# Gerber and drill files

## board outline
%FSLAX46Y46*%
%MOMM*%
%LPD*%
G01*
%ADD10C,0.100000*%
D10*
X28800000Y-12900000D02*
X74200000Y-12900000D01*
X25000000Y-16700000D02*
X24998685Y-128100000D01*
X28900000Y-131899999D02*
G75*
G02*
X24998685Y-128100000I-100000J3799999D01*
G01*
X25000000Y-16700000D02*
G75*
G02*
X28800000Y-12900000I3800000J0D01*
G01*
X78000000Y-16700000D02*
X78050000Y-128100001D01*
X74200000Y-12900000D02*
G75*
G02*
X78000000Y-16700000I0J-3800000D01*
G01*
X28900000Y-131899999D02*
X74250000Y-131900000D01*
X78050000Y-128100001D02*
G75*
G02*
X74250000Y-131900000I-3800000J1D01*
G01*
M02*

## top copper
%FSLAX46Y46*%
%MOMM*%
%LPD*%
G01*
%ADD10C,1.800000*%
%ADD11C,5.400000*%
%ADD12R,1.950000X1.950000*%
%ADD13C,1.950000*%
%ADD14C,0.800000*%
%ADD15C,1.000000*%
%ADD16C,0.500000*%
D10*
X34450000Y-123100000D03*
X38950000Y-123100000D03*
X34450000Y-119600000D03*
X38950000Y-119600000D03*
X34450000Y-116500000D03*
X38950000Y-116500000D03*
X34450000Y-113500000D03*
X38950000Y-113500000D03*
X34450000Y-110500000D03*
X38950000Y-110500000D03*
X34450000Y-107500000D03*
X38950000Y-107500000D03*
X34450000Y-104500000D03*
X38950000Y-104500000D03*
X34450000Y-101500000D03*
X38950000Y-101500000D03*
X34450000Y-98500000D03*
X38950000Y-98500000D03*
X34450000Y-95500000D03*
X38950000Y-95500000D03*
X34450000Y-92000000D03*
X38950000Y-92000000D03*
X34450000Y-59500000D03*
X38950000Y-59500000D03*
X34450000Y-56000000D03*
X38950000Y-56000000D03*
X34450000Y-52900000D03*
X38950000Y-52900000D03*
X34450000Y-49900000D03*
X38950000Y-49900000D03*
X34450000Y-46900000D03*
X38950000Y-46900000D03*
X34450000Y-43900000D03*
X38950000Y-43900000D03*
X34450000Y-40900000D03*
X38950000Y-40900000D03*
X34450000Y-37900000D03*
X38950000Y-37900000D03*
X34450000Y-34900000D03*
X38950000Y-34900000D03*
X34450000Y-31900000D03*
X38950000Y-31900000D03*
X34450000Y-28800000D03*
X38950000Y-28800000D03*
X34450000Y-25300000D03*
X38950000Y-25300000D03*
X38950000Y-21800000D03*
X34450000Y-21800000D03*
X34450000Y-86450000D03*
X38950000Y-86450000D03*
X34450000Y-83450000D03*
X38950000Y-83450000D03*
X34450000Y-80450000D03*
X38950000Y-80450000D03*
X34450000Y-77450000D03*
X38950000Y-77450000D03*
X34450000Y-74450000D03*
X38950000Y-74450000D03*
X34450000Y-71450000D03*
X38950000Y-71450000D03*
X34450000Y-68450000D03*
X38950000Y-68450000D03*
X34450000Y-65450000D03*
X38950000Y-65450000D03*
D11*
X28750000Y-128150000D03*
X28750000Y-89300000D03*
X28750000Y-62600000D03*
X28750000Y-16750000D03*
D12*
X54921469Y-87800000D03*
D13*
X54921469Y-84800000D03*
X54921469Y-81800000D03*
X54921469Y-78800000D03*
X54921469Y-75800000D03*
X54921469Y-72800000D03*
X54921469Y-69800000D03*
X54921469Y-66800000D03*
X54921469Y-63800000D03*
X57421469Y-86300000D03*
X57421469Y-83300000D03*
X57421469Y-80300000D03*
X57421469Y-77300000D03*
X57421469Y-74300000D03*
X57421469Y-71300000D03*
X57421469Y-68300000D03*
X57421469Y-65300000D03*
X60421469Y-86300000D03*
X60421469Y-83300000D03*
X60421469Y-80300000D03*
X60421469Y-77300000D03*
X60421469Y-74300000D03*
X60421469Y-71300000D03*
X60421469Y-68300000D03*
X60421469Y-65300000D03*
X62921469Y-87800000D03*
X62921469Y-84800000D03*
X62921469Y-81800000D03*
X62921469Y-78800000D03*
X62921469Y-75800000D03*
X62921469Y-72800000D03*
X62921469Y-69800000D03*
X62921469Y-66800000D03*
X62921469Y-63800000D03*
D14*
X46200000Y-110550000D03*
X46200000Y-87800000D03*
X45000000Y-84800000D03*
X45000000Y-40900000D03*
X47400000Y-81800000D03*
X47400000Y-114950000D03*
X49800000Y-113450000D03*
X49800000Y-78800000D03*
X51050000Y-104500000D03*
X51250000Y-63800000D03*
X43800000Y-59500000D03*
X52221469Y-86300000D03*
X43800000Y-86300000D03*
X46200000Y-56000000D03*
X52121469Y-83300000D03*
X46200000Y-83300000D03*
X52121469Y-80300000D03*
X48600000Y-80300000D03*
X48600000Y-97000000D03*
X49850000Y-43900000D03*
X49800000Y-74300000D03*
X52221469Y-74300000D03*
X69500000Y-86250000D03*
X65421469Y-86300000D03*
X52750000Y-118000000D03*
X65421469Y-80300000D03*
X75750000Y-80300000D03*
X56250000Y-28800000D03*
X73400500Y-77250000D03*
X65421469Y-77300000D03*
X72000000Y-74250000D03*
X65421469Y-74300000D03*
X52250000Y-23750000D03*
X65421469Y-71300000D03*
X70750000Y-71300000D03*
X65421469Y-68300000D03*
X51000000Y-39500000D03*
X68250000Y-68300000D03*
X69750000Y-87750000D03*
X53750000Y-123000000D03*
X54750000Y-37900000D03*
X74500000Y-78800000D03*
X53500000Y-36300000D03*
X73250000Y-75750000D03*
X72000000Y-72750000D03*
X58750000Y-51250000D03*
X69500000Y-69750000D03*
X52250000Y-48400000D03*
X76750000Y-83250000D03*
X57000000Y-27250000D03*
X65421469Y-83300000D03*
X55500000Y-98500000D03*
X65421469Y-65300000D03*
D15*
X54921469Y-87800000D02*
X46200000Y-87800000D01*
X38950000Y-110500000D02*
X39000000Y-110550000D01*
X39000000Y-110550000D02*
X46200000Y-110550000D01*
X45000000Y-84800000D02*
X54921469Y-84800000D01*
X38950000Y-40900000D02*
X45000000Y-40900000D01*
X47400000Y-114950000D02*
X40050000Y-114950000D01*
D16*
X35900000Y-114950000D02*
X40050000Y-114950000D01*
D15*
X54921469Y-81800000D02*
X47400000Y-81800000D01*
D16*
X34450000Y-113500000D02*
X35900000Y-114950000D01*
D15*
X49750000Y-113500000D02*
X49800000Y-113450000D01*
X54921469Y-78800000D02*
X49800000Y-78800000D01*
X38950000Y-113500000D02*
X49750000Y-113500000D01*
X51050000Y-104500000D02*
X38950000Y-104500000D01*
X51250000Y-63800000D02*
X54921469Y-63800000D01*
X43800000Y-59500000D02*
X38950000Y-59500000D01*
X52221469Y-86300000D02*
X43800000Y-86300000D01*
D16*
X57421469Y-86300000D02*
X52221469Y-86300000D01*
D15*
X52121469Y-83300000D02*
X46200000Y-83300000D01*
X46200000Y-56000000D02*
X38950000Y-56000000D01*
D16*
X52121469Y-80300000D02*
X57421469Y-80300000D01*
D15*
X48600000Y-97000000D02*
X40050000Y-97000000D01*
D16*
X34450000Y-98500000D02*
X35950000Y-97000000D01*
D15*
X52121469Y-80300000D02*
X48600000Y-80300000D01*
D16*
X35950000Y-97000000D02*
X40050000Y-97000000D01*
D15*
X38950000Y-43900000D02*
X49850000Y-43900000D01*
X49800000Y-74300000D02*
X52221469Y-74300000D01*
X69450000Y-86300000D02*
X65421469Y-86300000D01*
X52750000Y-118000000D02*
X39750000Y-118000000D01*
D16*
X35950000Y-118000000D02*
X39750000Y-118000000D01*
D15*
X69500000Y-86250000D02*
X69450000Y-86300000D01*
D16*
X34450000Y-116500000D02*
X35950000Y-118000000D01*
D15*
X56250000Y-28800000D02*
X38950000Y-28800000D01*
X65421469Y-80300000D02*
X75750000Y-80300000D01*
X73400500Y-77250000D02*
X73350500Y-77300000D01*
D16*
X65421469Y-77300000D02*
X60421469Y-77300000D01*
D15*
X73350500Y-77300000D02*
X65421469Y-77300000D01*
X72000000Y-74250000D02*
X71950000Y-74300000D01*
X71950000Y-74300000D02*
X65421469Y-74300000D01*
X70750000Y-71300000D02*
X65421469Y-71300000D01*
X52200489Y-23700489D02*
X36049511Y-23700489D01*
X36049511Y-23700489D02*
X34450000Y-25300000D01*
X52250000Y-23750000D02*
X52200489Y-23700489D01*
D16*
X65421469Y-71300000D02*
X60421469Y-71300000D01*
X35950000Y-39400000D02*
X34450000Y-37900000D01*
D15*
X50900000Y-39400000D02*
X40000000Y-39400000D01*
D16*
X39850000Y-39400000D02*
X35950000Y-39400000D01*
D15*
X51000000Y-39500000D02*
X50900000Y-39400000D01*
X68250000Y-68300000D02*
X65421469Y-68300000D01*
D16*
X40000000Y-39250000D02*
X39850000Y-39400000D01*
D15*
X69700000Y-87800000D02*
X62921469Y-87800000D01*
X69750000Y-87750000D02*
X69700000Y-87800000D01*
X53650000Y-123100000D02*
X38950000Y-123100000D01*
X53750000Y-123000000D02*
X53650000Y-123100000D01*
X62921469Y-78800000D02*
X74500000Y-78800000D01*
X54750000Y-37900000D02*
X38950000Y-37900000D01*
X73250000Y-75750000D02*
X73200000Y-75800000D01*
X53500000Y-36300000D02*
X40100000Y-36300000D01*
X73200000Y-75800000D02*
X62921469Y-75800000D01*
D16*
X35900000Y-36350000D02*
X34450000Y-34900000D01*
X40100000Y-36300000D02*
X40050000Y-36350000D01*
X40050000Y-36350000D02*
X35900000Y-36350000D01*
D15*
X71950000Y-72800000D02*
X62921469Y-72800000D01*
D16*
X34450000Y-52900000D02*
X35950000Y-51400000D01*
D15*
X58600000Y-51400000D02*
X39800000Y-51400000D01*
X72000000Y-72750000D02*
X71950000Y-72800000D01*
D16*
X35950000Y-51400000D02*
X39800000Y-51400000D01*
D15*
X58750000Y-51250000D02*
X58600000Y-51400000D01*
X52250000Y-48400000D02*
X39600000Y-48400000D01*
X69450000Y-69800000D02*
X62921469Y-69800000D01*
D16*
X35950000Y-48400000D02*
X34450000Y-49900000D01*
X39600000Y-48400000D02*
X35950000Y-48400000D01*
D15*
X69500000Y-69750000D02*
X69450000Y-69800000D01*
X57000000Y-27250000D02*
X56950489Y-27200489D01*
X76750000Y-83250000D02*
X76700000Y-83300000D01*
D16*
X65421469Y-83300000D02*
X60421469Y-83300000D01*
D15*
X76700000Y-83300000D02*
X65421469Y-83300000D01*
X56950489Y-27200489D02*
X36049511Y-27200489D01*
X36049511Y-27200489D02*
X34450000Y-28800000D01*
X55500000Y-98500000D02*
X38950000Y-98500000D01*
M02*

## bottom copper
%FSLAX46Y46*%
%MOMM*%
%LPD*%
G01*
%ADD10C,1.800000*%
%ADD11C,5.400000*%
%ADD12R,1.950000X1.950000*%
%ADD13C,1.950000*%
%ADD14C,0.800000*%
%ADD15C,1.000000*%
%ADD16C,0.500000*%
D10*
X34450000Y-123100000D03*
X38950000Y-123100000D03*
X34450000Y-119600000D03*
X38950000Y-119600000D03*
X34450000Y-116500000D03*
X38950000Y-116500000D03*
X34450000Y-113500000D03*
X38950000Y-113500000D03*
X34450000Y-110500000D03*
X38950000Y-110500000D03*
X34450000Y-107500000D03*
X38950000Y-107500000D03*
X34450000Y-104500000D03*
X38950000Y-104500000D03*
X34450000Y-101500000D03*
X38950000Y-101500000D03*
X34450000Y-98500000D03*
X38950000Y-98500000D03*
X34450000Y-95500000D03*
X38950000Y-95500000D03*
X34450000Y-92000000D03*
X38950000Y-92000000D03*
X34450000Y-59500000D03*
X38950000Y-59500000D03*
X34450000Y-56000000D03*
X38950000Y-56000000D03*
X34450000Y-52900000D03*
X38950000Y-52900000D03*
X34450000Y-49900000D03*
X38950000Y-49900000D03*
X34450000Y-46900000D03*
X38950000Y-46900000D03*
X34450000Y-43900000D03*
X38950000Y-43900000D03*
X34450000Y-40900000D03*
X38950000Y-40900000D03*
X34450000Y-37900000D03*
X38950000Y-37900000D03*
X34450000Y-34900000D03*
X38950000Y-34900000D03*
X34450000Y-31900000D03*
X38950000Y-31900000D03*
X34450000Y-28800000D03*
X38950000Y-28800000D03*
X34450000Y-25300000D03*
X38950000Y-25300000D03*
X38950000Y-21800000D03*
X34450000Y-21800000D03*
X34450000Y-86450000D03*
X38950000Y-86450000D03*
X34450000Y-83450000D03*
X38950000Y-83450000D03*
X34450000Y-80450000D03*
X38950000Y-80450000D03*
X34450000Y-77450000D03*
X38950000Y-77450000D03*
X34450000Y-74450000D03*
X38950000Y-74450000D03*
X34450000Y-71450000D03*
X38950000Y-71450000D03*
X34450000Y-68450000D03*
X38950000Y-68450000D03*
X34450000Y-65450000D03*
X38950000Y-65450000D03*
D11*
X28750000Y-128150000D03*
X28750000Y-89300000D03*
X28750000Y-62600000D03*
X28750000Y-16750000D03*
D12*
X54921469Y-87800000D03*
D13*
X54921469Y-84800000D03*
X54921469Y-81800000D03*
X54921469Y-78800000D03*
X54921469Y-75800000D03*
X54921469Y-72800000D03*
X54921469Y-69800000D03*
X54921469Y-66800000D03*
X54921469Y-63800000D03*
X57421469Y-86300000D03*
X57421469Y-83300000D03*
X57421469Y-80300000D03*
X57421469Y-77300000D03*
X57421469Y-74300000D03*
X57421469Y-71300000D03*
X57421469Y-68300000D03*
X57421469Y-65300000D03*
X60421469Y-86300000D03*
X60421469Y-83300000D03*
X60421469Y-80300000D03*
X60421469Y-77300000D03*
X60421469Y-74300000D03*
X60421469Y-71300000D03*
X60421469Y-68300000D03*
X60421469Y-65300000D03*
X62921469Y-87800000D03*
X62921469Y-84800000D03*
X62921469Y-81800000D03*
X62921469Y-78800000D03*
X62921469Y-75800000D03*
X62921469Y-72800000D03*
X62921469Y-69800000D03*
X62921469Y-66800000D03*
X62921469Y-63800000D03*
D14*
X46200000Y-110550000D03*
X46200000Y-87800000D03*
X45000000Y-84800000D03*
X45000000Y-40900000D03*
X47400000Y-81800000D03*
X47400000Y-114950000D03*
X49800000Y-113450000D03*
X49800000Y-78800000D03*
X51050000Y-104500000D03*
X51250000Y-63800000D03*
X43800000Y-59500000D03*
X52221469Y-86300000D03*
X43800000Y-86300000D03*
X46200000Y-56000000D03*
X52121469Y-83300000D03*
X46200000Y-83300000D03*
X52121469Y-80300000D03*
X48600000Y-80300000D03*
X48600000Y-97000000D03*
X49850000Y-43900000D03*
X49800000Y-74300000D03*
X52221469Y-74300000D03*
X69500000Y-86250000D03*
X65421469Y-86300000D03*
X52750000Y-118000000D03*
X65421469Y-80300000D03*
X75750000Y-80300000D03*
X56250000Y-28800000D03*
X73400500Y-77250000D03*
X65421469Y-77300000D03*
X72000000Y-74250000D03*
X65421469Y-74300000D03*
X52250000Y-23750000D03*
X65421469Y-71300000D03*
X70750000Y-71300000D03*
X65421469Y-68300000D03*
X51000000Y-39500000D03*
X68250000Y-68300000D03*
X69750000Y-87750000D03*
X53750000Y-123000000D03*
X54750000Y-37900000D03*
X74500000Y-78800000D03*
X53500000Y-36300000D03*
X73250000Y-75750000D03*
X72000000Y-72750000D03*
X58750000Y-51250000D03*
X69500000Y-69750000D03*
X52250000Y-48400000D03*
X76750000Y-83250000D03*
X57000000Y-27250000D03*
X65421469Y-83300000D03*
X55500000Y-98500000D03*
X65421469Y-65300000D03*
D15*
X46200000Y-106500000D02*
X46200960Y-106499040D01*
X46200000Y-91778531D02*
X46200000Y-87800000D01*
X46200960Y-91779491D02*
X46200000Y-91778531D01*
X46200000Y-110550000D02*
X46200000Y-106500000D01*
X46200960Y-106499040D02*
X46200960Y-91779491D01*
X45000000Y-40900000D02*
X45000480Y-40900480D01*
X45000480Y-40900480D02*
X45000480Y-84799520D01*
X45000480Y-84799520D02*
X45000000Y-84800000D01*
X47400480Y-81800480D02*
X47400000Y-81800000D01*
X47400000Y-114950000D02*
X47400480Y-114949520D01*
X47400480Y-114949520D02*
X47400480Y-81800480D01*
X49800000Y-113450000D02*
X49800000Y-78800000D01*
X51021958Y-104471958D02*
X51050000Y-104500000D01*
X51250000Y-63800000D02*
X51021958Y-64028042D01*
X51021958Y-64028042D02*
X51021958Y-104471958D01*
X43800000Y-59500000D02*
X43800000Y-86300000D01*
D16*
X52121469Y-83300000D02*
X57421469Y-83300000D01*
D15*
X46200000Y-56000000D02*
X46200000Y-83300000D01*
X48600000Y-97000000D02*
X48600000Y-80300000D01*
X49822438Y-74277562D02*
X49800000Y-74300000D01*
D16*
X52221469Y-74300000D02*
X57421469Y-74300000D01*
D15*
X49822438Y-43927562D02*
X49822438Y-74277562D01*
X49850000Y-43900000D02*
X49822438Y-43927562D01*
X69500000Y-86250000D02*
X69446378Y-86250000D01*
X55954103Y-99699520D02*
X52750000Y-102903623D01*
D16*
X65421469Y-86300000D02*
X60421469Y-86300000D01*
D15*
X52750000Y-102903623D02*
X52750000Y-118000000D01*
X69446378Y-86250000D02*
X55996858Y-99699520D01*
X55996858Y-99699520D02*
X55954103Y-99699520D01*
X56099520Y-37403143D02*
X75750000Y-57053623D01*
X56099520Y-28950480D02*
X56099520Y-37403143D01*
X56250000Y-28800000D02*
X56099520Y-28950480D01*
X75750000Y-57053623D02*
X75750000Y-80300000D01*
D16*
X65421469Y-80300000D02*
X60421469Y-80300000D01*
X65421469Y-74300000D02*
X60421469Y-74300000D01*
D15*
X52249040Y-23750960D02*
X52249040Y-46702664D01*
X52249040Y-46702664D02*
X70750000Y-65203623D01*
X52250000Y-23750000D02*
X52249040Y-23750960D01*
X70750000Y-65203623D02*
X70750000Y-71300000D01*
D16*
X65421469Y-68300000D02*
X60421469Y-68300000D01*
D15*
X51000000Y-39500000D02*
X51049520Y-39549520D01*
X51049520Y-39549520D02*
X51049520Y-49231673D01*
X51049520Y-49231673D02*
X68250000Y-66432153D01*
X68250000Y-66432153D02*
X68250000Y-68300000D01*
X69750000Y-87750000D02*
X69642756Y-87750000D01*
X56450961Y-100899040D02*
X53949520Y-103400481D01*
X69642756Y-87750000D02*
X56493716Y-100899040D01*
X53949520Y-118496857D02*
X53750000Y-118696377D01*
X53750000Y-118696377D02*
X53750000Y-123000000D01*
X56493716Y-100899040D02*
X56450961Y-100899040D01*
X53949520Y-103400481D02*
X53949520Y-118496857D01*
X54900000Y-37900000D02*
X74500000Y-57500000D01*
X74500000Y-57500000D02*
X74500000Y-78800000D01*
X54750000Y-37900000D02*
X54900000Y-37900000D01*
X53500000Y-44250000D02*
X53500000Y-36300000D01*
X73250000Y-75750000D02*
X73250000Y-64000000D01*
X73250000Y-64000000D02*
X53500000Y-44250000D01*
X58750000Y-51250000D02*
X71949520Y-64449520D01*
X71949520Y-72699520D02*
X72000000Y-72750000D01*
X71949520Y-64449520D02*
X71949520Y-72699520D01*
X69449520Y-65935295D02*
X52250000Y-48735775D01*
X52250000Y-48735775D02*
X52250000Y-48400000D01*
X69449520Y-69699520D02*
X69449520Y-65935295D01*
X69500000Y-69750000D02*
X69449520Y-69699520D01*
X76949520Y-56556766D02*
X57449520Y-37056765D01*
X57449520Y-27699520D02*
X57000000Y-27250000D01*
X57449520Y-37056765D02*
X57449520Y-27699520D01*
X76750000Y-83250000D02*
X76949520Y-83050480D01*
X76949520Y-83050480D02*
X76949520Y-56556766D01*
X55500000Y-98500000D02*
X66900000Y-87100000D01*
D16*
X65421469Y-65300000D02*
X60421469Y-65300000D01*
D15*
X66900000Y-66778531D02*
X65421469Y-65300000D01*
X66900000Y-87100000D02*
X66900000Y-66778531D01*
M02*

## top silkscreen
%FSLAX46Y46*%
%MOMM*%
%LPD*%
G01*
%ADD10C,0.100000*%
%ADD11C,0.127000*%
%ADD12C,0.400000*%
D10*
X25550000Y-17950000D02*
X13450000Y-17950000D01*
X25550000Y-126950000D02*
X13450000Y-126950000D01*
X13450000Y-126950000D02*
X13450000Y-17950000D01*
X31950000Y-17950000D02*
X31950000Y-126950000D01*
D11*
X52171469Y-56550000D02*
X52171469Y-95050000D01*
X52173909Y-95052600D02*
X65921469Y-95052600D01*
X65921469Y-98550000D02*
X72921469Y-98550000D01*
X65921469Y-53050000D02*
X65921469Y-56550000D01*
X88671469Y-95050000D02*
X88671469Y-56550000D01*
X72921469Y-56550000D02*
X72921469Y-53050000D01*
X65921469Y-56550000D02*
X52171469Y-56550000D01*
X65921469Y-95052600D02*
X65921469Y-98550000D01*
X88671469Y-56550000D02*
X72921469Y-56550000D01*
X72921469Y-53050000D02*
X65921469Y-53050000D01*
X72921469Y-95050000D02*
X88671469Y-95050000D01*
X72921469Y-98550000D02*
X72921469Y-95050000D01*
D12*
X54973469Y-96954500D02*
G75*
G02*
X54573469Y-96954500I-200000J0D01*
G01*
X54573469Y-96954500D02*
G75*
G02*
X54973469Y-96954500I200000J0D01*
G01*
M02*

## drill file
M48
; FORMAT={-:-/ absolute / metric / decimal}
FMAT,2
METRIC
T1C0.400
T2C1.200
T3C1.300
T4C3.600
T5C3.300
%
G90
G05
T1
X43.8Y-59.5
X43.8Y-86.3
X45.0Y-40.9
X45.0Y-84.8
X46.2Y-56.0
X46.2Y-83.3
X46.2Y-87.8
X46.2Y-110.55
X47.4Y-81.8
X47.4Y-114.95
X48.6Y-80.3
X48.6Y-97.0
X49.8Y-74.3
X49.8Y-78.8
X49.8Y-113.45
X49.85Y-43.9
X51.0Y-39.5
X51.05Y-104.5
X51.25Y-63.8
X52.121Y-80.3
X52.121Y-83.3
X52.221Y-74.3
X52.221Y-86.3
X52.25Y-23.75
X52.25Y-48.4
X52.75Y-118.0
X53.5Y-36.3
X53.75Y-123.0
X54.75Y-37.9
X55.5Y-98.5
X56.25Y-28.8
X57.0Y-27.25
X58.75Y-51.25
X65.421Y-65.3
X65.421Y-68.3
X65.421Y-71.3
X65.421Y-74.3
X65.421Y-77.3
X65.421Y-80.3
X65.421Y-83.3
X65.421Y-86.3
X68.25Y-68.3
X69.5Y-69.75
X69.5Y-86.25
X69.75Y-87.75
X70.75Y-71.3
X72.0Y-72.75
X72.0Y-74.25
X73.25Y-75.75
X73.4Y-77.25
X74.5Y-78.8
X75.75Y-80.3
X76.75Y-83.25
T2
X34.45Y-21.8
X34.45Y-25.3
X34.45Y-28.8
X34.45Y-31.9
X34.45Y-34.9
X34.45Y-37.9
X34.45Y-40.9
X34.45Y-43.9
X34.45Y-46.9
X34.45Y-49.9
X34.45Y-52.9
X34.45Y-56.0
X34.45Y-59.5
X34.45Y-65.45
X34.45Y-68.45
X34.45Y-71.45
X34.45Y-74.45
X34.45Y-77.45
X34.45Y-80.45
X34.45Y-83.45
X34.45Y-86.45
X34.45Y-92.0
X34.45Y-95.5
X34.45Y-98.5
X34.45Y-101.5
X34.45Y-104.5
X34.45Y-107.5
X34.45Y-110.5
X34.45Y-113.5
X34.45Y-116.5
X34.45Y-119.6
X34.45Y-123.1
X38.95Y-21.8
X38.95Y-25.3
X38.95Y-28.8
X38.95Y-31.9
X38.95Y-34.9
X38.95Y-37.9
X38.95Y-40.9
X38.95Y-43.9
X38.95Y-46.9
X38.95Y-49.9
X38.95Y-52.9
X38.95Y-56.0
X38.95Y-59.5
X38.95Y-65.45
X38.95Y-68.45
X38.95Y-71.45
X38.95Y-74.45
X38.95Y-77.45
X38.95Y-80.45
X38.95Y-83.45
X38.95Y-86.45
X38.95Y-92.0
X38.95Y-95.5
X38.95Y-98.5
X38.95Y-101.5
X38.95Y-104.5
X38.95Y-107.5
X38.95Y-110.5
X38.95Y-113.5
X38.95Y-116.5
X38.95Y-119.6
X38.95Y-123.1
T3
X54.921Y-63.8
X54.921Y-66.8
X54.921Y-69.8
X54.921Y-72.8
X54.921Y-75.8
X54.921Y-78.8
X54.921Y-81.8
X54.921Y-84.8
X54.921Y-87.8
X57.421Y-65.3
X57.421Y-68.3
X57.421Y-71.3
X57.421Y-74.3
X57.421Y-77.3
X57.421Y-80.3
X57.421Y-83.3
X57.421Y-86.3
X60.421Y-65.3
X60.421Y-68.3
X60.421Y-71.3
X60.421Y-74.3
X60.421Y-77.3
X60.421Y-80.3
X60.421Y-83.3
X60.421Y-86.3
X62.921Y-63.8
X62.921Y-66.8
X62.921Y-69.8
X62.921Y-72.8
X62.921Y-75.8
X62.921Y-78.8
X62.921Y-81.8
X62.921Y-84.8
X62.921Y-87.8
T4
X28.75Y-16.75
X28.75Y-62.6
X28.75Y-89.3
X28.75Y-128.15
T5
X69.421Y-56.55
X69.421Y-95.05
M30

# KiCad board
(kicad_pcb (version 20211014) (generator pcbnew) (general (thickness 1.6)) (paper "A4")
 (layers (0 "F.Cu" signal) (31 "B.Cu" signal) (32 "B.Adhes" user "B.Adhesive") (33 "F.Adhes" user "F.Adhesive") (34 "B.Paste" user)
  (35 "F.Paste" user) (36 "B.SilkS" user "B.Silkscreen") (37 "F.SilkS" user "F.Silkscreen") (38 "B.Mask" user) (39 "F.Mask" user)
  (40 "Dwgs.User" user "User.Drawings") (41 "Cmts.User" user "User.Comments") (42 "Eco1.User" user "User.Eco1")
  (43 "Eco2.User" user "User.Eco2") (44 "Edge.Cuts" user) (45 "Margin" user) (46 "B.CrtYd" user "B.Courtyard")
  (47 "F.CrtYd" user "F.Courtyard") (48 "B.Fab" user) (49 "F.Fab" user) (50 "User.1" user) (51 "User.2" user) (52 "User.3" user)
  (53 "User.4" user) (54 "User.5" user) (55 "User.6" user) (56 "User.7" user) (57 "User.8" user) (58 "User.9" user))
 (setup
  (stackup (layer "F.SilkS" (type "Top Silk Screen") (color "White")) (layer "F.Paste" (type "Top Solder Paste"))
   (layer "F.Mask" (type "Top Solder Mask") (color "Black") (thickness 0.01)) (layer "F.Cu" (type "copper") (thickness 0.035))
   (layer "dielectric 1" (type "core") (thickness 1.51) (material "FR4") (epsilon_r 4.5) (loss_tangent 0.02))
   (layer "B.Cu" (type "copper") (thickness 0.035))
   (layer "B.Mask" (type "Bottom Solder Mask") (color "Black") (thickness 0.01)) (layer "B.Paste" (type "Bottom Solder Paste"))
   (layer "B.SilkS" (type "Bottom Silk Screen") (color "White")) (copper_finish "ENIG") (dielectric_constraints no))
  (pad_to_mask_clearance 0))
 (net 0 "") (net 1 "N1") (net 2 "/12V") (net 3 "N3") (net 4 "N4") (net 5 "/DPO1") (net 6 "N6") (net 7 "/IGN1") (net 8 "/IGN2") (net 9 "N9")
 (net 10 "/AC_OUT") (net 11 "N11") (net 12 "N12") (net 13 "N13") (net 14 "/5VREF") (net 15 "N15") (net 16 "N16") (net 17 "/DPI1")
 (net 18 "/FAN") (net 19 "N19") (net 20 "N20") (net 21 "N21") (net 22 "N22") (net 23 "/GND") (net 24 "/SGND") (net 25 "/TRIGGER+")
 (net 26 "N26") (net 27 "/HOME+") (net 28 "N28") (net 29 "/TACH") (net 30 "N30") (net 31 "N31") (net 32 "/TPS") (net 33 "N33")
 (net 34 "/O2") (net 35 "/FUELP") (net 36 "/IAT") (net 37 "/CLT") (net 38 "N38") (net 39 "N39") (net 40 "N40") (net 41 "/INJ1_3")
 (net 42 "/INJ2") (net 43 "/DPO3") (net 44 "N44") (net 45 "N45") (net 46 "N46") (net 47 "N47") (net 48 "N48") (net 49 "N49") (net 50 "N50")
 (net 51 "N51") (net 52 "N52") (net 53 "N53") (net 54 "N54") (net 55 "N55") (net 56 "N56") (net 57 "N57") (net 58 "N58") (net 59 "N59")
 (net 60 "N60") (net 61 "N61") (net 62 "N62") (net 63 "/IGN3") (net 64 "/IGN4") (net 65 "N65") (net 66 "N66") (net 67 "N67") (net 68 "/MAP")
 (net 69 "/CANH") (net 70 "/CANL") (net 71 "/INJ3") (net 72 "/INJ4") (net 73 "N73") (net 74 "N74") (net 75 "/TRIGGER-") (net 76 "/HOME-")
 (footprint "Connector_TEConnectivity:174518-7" (layer "F.Cu") (at 27.45 72.8 90)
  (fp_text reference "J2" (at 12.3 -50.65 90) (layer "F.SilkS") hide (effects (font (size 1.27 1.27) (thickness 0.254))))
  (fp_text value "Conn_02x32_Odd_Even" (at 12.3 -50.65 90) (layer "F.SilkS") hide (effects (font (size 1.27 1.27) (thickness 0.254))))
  (fp_line (start 54.85 -1.9) (end 54.85 -14) (layer "F.SilkS") (width 0.1))
  (fp_line (start -54.15 -1.9) (end -54.15 -14) (layer "F.SilkS") (width 0.1))
  (fp_line (start -54.15 -14) (end 54.85 -14) (layer "F.SilkS") (width 0.1))
  (fp_line (start 54.85 4.5) (end -54.15 4.5) (layer "F.SilkS") (width 0.1))
  (pad "1A" thru_hole circle (at -50.3 7 180) (size 1.8 1.8) (drill 1.2) (layers *.Cu *.Mask) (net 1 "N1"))
  (pad "1B" thru_hole circle (at -50.3 11.5 180) (size 1.8 1.8) (drill 1.2) (layers *.Cu *.Mask) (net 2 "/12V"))
  (pad "1C" thru_hole circle (at -46.8 7 180) (size 1.8 1.8) (drill 1.2) (layers *.Cu *.Mask) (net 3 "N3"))
  (pad "1D" thru_hole circle (at -46.8 11.5 180) (size 1.8 1.8) (drill 1.2) (layers *.Cu *.Mask) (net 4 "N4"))
  (pad "1E" thru_hole circle (at -43.7 7 180) (size 1.8 1.8) (drill 1.2) (layers *.Cu *.Mask) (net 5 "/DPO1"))
  (pad "1F" thru_hole circle (at -43.7 11.5 180) (size 1.8 1.8) (drill 1.2) (layers *.Cu *.Mask) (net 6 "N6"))
  (pad "1G" thru_hole circle (at -40.7 7 180) (size 1.8 1.8) (drill 1.2) (layers *.Cu *.Mask) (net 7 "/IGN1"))
  (pad "1H" thru_hole circle (at -40.7 11.5 180) (size 1.8 1.8) (drill 1.2) (layers *.Cu *.Mask) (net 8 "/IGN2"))
  (pad "1I" thru_hole circle (at -37.7 7 180) (size 1.8 1.8) (drill 1.2) (layers *.Cu *.Mask) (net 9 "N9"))
  (pad "1J" thru_hole circle (at -37.7 11.5 180) (size 1.8 1.8) (drill 1.2) (layers *.Cu *.Mask) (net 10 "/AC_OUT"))
  (pad "1K" thru_hole circle (at -34.7 7 180) (size 1.8 1.8) (drill 1.2) (layers *.Cu *.Mask) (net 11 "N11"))
  (pad "1L" thru_hole circle (at -34.7 11.5 180) (size 1.8 1.8) (drill 1.2) (layers *.Cu *.Mask) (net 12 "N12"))
  (pad "1M" thru_hole circle (at -31.7 7 180) (size 1.8 1.8) (drill 1.2) (layers *.Cu *.Mask) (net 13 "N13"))
  (pad "1N" thru_hole circle (at -31.7 11.5 180) (size 1.8 1.8) (drill 1.2) (layers *.Cu *.Mask) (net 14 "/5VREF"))
  (pad "1O" thru_hole circle (at -28.7 7 180) (size 1.8 1.8) (drill 1.2) (layers *.Cu *.Mask) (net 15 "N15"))
  (pad "1P" thru_hole circle (at -28.7 11.5 180) (size 1.8 1.8) (drill 1.2) (layers *.Cu *.Mask) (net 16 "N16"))
  (pad "1Q" thru_hole circle (at -25.7 7 180) (size 1.8 1.8) (drill 1.2) (layers *.Cu *.Mask) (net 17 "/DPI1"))
  (pad "1R" thru_hole circle (at -25.7 11.5 180) (size 1.8 1.8) (drill 1.2) (layers *.Cu *.Mask) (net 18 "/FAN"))
  (pad "1S" thru_hole circle (at -22.7 7 180) (size 1.8 1.8) (drill 1.2) (layers *.Cu *.Mask) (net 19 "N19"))
  (pad "1T" thru_hole circle (at -22.7 11.5 180) (size 1.8 1.8) (drill 1.2) (layers *.Cu *.Mask) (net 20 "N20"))
  (pad "1U" thru_hole circle (at -19.2 7 180) (size 1.8 1.8) (drill 1.2) (layers *.Cu *.Mask) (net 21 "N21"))
  (pad "1V" thru_hole circle (at -19.2 11.5 180) (size 1.8 1.8) (drill 1.2) (layers *.Cu *.Mask) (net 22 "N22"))
  (pad "2A" thru_hole circle (at 13.3 7 180) (size 1.8 1.8) (drill 1.2) (layers *.Cu *.Mask) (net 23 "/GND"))
  (pad "2B" thru_hole circle (at 13.3 11.5 180) (size 1.8 1.8) (drill 1.2) (layers *.Cu *.Mask) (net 23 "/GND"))
  (pad "2C" thru_hole circle (at 16.8 7 180) (size 1.8 1.8) (drill 1.2) (layers *.Cu *.Mask) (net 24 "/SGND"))
  (pad "2D" thru_hole circle (at 16.8 11.5 180) (size 1.8 1.8) (drill 1.2) (layers *.Cu *.Mask) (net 24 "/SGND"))
  (pad "2E" thru_hole circle (at 19.9 7 180) (size 1.8 1.8) (drill 1.2) (layers *.Cu *.Mask) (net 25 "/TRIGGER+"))
  (pad "2F" thru_hole circle (at 19.9 11.5 180) (size 1.8 1.8) (drill 1.2) (layers *.Cu *.Mask) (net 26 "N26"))
  (pad "2G" thru_hole circle (at 22.9 7 180) (size 1.8 1.8) (drill 1.2) (layers *.Cu *.Mask) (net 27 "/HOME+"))
  (pad "2H" thru_hole circle (at 22.9 11.5 180) (size 1.8 1.8) (drill 1.2) (layers *.Cu *.Mask) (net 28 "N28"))
  (pad "2I" thru_hole circle (at 25.9 7 180) (size 1.8 1.8) (drill 1.2) (layers *.Cu *.Mask) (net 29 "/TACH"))
  (pad "2J" thru_hole circle (at 25.9 11.5 180) (size 1.8 1.8) (drill 1.2) (layers *.Cu *.Mask) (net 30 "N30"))
  (pad "2K" thru_hole circle (at 28.9 7 180) (size 1.8 1.8) (drill 1.2) (layers *.Cu *.Mask) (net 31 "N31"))
  (pad "2L" thru_hole circle (at 28.9 11.5 180) (size 1.8 1.8) (drill 1.2) (layers *.Cu *.Mask) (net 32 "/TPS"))
  (pad "2M" thru_hole circle (at 31.9 7 180) (size 1.8 1.8) (drill 1.2) (layers *.Cu *.Mask) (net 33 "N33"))
  (pad "2N" thru_hole circle (at 31.9 11.5 180) (size 1.8 1.8) (drill 1.2) (layers *.Cu *.Mask) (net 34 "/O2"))
  (pad "2O" thru_hole circle (at 34.9 7 180) (size 1.8 1.8) (drill 1.2) (layers *.Cu *.Mask) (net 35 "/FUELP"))
  (pad "2P" thru_hole circle (at 34.9 11.5 180) (size 1.8 1.8) (drill 1.2) (layers *.Cu *.Mask) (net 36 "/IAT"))
  (pad "2Q" thru_hole circle (at 37.9 7 180) (size 1.8 1.8) (drill 1.2) (layers *.Cu *.Mask) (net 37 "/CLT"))
  (pad "2R" thru_hole circle (at 37.9 11.5 180) (size 1.8 1.8) (drill 1.2) (layers *.Cu *.Mask) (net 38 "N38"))
  (pad "2S" thru_hole circle (at 40.9 7 180) (size 1.8 1.8) (drill 1.2) (layers *.Cu *.Mask) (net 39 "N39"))
  (pad "2T" thru_hole circle (at 40.9 11.5 180) (size 1.8 1.8) (drill 1.2) (layers *.Cu *.Mask) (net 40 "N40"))
  (pad "2U" thru_hole circle (at 44 7 180) (size 1.8 1.8) (drill 1.2) (layers *.Cu *.Mask) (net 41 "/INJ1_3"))
  (pad "2V" thru_hole circle (at 44 11.5 180) (size 1.8 1.8) (drill 1.2) (layers *.Cu *.Mask) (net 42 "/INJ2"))
  (pad "2W" thru_hole circle (at 47.5 7 180) (size 1.8 1.8) (drill 1.2) (layers *.Cu *.Mask) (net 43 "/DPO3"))
  (pad "2X" thru_hole circle (at 47.5 11.5 180) (size 1.8 1.8) (drill 1.2) (layers *.Cu *.Mask) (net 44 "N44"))
  (pad "2Y" thru_hole circle (at 51 11.5 180) (size 1.8 1.8) (drill 1.2) (layers *.Cu *.Mask) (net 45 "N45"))
  (pad "2Z" thru_hole circle (at 51 7 180) (size 1.8 1.8) (drill 1.2) (layers *.Cu *.Mask) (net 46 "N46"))
  (pad "3A" thru_hole circle (at -13.65 7 180) (size 1.8 1.8) (drill 1.2) (layers *.Cu *.Mask) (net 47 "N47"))
  (pad "3B" thru_hole circle (at -13.65 11.5 180) (size 1.8 1.8) (drill 1.2) (layers *.Cu *.Mask) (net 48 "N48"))
  (pad "3C" thru_hole circle (at -10.65 7 180) (size 1.8 1.8) (drill 1.2) (layers *.Cu *.Mask) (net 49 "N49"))
  (pad "3D" thru_hole circle (at -10.65 11.5 180) (size 1.8 1.8) (drill 1.2) (layers *.Cu *.Mask) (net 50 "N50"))
  (pad "3E" thru_hole circle (at -7.65 7 180) (size 1.8 1.8) (drill 1.2) (layers *.Cu *.Mask) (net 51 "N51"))
  (pad "3F" thru_hole circle (at -7.65 11.5 180) (size 1.8 1.8) (drill 1.2) (layers *.Cu *.Mask) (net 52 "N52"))
  (pad "3G" thru_hole circle (at -4.65 7 180) (size 1.8 1.8) (drill 1.2) (layers *.Cu *.Mask) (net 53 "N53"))
  (pad "3H" thru_hole circle (at -4.65 11.5 180) (size 1.8 1.8) (drill 1.2) (layers *.Cu *.Mask) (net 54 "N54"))
  (pad "3I" thru_hole circle (at -1.65 7 180) (size 1.8 1.8) (drill 1.2) (layers *.Cu *.Mask) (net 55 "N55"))
  (pad "3J" thru_hole circle (at -1.65 11.5 180) (size 1.8 1.8) (drill 1.2) (layers *.Cu *.Mask) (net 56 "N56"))
  (pad "3K" thru_hole circle (at 1.35 7 180) (size 1.8 1.8) (drill 1.2) (layers *.Cu *.Mask) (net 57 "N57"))
  (pad "3L" thru_hole circle (at 1.35 11.5 180) (size 1.8 1.8) (drill 1.2) (layers *.Cu *.Mask) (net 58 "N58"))
  (pad "3M" thru_hole circle (at 4.35 7 180) (size 1.8 1.8) (drill 1.2) (layers *.Cu *.Mask) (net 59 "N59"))
  (pad "3N" thru_hole circle (at 4.35 11.5 180) (size 1.8 1.8) (drill 1.2) (layers *.Cu *.Mask) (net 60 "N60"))
  (pad "3O" thru_hole circle (at 7.35 7 180) (size 1.8 1.8) (drill 1.2) (layers *.Cu *.Mask) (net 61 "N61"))
  (pad "3P" thru_hole circle (at 7.35 11.5 180) (size 1.8 1.8) (drill 1.2) (layers *.Cu *.Mask) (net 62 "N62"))
  (pad "MH1" thru_hole circle (at -55.35 1.3 180) (size 5.4 5.4) (drill 3.6) (layers *.Cu *.Mask))
  (pad "MH2" thru_hole circle (at -16.5 1.3 180) (size 5.4 5.4) (drill 3.6) (layers *.Cu *.Mask))
  (pad "MH3" thru_hole circle (at 10.2 1.3 180) (size 5.4 5.4) (drill 3.6) (layers *.Cu *.Mask))
  (pad "MH4" thru_hole circle (at 56.05 1.3 180) (size 5.4 5.4) (drill 3.6) (layers *.Cu *.Mask)))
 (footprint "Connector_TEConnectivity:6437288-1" (layer "F.Cu") (at 58.921469 75.8 90)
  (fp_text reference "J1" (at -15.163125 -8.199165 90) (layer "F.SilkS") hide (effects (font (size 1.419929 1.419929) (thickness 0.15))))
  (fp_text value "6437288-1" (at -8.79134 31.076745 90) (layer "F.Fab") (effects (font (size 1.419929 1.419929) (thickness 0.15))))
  (fp_line (start 19.25 -6.75) (end -19.25 -6.75) (layer "F.SilkS") (width 0.127))
  (fp_line (start -19.2526 -6.74756) (end -19.2526 7) (layer "F.SilkS") (width 0.127))
  (fp_line (start -22.75 7) (end -22.75 14) (layer "F.SilkS") (width 0.127))
  (fp_line (start 22.75 7) (end 19.25 7) (layer "F.SilkS") (width 0.127))
  (fp_line (start -19.25 29.75) (end 19.25 29.75) (layer "F.SilkS") (width 0.127))
  (fp_line (start 19.25 14) (end 22.75 14) (layer "F.SilkS") (width 0.127))
  (fp_line (start 19.25 7) (end 19.25 -6.75) (layer "F.SilkS") (width 0.127))
  (fp_line (start -19.2526 7) (end -22.75 7) (layer "F.SilkS") (width 0.127))
  (fp_line (start 19.25 29.75) (end 19.25 14) (layer "F.SilkS") (width 0.127))
  (fp_line (start 22.75 14) (end 22.75 7) (layer "F.SilkS") (width 0.127))
  (fp_line (start -19.25 14) (end -19.25 29.75) (layer "F.SilkS") (width 0.127))
  (fp_line (start -22.75 14) (end -19.25 14) (layer "F.SilkS") (width 0.127))
  (fp_circle (center -21.1545 -4.148) (end -20.9545 -4.148) (layer "F.SilkS") (width 0.4) (fill none))
  (pad "" np_thru_hole circle (at -19.25 10.5 90) (size 3.3 3.3) (drill 3.3) (layers *.Cu *.Mask))
  (pad "" np_thru_hole circle (at 19.25 10.5 90) (size 3.3 3.3) (drill 3.3) (layers *.Cu *.Mask))
  (pad "1" thru_hole rect (at -12 -4 90) (size 1.95 1.95) (drill 1.3) (layers *.Cu *.Mask) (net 10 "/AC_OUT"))
  (pad "2" thru_hole circle (at -9 -4 90) (size 1.95 1.95) (drill 1.3) (layers *.Cu *.Mask) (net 34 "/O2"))
  (pad "3" thru_hole circle (at -6 -4 90) (size 1.95 1.95) (drill 1.3) (layers *.Cu *.Mask) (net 7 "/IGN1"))
  (pad "4" thru_hole circle (at -3 -4 90) (size 1.95 1.95) (drill 1.3) (layers *.Cu *.Mask) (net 8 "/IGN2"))
  (pad "5" thru_hole circle (at 0 -4 90) (size 1.95 1.95) (drill 1.3) (layers *.Cu *.Mask) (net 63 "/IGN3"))
  (pad "6" thru_hole circle (at 3 -4 90) (size 1.95 1.95) (drill 1.3) (layers *.Cu *.Mask) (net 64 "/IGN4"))
  (pad "7" thru_hole circle (at 6 -4 90) (size 1.95 1.95) (drill 1.3) (layers *.Cu *.Mask) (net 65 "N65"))
  (pad "8" thru_hole circle (at 9 -4 90) (size 1.95 1.95) (drill 1.3) (layers *.Cu *.Mask) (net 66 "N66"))
  (pad "9" thru_hole circle (at 12 -4 90) (size 1.95 1.95) (drill 1.3) (layers *.Cu *.Mask) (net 14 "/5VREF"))
  (pad "10" thru_hole circle (at -10.5 -1.5 90) (size 1.95 1.95) (drill 1.3) (layers *.Cu *.Mask) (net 23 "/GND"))
  (pad "11" thru_hole circle (at -7.5 -1.5 90) (size 1.95 1.95) (drill 1.3) (layers *.Cu *.Mask) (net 24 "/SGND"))
  (pad "12" thru_hole circle (at -4.5 -1.5 90) (size 1.95 1.95) (drill 1.3) (layers *.Cu *.Mask) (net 17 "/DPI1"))
  (pad "13" thru_hole circle (at -1.5 -1.5 90) (size 1.95 1.95) (drill 1.3) (layers *.Cu *.Mask) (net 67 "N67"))
  (pad "14" thru_hole circle (at 1.5 -1.5 90) (size 1.95 1.95) (drill 1.3) (layers *.Cu *.Mask) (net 32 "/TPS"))
  (pad "15" thru_hole circle (at 4.5 -1.5 90) (size 1.95 1.95) (drill 1.3) (layers *.Cu *.Mask) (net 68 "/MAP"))
  (pad "16" thru_hole circle (at 7.5 -1.5 90) (size 1.95 1.95) (drill 1.3) (layers *.Cu *.Mask) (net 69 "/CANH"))
  (pad "17" thru_hole circle (at 10.5 -1.5 90) (size 1.95 1.95) (drill 1.3) (layers *.Cu *.Mask) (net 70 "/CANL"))
  (pad "18" thru_hole circle (at -10.5 1.5 90) (size 1.95 1.95) (drill 1.3) (layers *.Cu *.Mask) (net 5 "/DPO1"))
  (pad "19" thru_hole circle (at -7.5 1.5 90) (size 1.95 1.95) (drill 1.3) (layers *.Cu *.Mask) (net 41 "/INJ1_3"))
  (pad "20" thru_hole circle (at -4.5 1.5 90) (size 1.95 1.95) (drill 1.3) (layers *.Cu *.Mask) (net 42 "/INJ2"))
  (pad "21" thru_hole circle (at -1.5 1.5 90) (size 1.95 1.95) (drill 1.3) (layers *.Cu *.Mask) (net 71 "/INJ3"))
  (pad "22" thru_hole circle (at 1.5 1.5 90) (size 1.95 1.95) (drill 1.3) (layers *.Cu *.Mask) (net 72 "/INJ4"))
  (pad "23" thru_hole circle (at 4.5 1.5 90) (size 1.95 1.95) (drill 1.3) (layers *.Cu *.Mask) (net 43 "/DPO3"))
  (pad "24" thru_hole circle (at 7.5 1.5 90) (size 1.95 1.95) (drill 1.3) (layers *.Cu *.Mask) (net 35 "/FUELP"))
  (pad "25" thru_hole circle (at 10.5 1.5 90) (size 1.95 1.95) (drill 1.3) (layers *.Cu *.Mask) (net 18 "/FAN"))
  (pad "26" thru_hole circle (at -12 4 90) (size 1.95 1.95) (drill 1.3) (layers *.Cu *.Mask) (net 2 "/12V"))
  (pad "27" thru_hole circle (at -9 4 90) (size 1.95 1.95) (drill 1.3) (layers *.Cu *.Mask) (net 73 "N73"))
  (pad "28" thru_hole circle (at -6 4 90) (size 1.95 1.95) (drill 1.3) (layers *.Cu *.Mask) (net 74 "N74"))
  (pad "29" thru_hole circle (at -3 4 90) (size 1.95 1.95) (drill 1.3) (layers *.Cu *.Mask) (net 36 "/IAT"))
  (pad "30" thru_hole circle (at 0 4 90) (size 1.95 1.95) (drill 1.3) (layers *.Cu *.Mask) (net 37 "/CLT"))
  (pad "31" thru_hole circle (at 3 4 90) (size 1.95 1.95) (drill 1.3) (layers *.Cu *.Mask) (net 25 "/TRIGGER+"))
  (pad "32" thru_hole circle (at 6 4 90) (size 1.95 1.95) (drill 1.3) (layers *.Cu *.Mask) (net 27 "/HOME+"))
  (pad "33" thru_hole circle (at 9 4 90) (size 1.95 1.95) (drill 1.3) (layers *.Cu *.Mask) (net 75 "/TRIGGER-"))
  (pad "34" thru_hole circle (at 12 4 90) (size 1.95 1.95) (drill 1.3) (layers *.Cu *.Mask) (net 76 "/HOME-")))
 (gr_line (start 28.8 12.9) (end 74.2 12.9) (layer "Edge.Cuts") (width 0.1))
 (gr_line (start 25 16.7) (end 24.998685 128.1) (layer "Edge.Cuts") (width 0.1))
 (gr_arc (start 28.9 131.899999) (mid 26.147656 130.823061) (end 24.998685 128.1) (layer "Edge.Cuts") (width 0.1))
 (gr_arc (start 25 16.7) (mid 26.112994 14.012994) (end 28.8 12.9) (layer "Edge.Cuts") (width 0.1))
 (gr_line (start 78 16.7) (end 78.05 128.100001) (layer "Edge.Cuts") (width 0.1))
 (gr_arc (start 74.2 12.9) (mid 76.887006 14.012994) (end 78 16.7) (layer "Edge.Cuts") (width 0.1))
 (gr_line (start 28.9 131.899999) (end 74.25 131.9) (layer "Edge.Cuts") (width 0.1))
 (gr_arc (start 78.05 128.100001) (mid 76.937006 130.787006) (end 74.25 131.9) (layer "Edge.Cuts") (width 0.1))
 (segment (start 54.921469 87.8) (end 46.2 87.8) (width 1) (layer "F.Cu") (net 10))
 (segment (start 38.95 110.5) (end 39 110.55) (width 1) (layer "F.Cu") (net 10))
 (segment (start 39 110.55) (end 46.2 110.55) (width 1) (layer "F.Cu") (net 10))
 (via (at 46.2 110.55) (size 0.8) (drill 0.4) (layers "F.Cu" "B.Cu") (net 10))
 (via (at 46.2 87.8) (size 0.8) (drill 0.4) (layers "F.Cu" "B.Cu") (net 10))
 (segment (start 46.2 106.5) (end 46.20096 106.49904) (width 1) (layer "B.Cu") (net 10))
 (segment (start 46.2 91.778531) (end 46.2 87.8) (width 1) (layer "B.Cu") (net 10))
 (segment (start 46.20096 91.779491) (end 46.2 91.778531) (width 1) (layer "B.Cu") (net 10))
 (segment (start 46.2 110.55) (end 46.2 106.5) (width 1) (layer "B.Cu") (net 10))
 (segment (start 46.20096 106.49904) (end 46.20096 91.779491) (width 1) (layer "B.Cu") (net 10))
 (segment (start 45 84.8) (end 54.921469 84.8) (width 1) (layer "F.Cu") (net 34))
 (segment (start 38.95 40.9) (end 45 40.9) (width 1) (layer "F.Cu") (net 34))
 (via (at 45 84.8) (size 0.8) (drill 0.4) (layers "F.Cu" "B.Cu") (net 34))
 (via (at 45 40.9) (size 0.8) (drill 0.4) (layers "F.Cu" "B.Cu") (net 34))
 (segment (start 45 40.9) (end 45.00048 40.90048) (width 1) (layer "B.Cu") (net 34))
 (segment (start 45.00048 40.90048) (end 45.00048 84.79952) (width 1) (layer "B.Cu") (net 34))
 (segment (start 45.00048 84.79952) (end 45 84.8) (width 1) (layer "B.Cu") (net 34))
 (segment (start 47.4 114.95) (end 40.05 114.95) (width 1) (layer "F.Cu") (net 7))
 (segment (start 35.9 114.95) (end 40.05 114.95) (width 0.5) (layer "F.Cu") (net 7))
 (segment (start 54.921469 81.8) (end 47.4 81.8) (width 1) (layer "F.Cu") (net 7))
 (segment (start 34.45 113.5) (end 35.9 114.95) (width 0.5) (layer "F.Cu") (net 7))
 (via (at 47.4 81.8) (size 0.8) (drill 0.4) (layers "F.Cu" "B.Cu") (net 7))
 (via (at 47.4 114.95) (size 0.8) (drill 0.4) (layers "F.Cu" "B.Cu") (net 7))
 (segment (start 47.40048 81.80048) (end 47.4 81.8) (width 1) (layer "B.Cu") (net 7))
 (segment (start 47.4 114.95) (end 47.40048 114.94952) (width 1) (layer "B.Cu") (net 7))
 (segment (start 47.40048 114.94952) (end 47.40048 81.80048) (width 1) (layer "B.Cu") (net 7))
 (segment (start 49.75 113.5) (end 49.8 113.45) (width 1) (layer "F.Cu") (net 8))
 (segment (start 54.921469 78.8) (end 49.8 78.8) (width 1) (layer "F.Cu") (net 8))
 (segment (start 38.95 113.5) (end 49.75 113.5) (width 1) (layer "F.Cu") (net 8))
 (via (at 49.8 113.45) (size 0.8) (drill 0.4) (layers "F.Cu" "B.Cu") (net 8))
 (via (at 49.8 78.8) (size 0.8) (drill 0.4) (layers "F.Cu" "B.Cu") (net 8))
 (segment (start 49.8 113.45) (end 49.8 78.8) (width 1) (layer "B.Cu") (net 8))
 (segment (start 51.05 104.5) (end 38.95 104.5) (width 1) (layer "F.Cu") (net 14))
 (segment (start 51.25 63.8) (end 54.921469 63.8) (width 1) (layer "F.Cu") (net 14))
 (via (at 51.05 104.5) (size 0.8) (drill 0.4) (layers "F.Cu" "B.Cu") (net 14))
 (via (at 51.25 63.8) (size 0.8) (drill 0.4) (layers "F.Cu" "B.Cu") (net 14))
 (segment (start 51.021958 104.471958) (end 51.05 104.5) (width 1) (layer "B.Cu") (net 14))
 (segment (start 51.25 63.8) (end 51.021958 64.028042) (width 1) (layer "B.Cu") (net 14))
 (segment (start 51.021958 64.028042) (end 51.021958 104.471958) (width 1) (layer "B.Cu") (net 14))
 (segment (start 43.8 59.5) (end 38.95 59.5) (width 1) (layer "F.Cu") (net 23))
 (segment (start 52.221469 86.3) (end 43.8 86.3) (width 1) (layer "F.Cu") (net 23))
 (segment (start 57.421469 86.3) (end 52.221469 86.3) (width 0.5) (layer "F.Cu") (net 23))
 (via (at 43.8 59.5) (size 0.8) (drill 0.4) (layers "F.Cu" "B.Cu") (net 23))
 (via (at 52.221469 86.3) (size 0.8) (drill 0.4) (layers "F.Cu" "B.Cu") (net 23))
 (via (at 43.8 86.3) (size 0.8) (drill 0.4) (layers "F.Cu" "B.Cu") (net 23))
 (segment (start 43.8 59.5) (end 43.8 86.3) (width 1) (layer "B.Cu") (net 23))
 (segment (start 52.121469 83.3) (end 46.2 83.3) (width 1) (layer "F.Cu") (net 24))
 (segment (start 46.2 56) (end 38.95 56) (width 1) (layer "F.Cu") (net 24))
 (via (at 46.2 56) (size 0.8) (drill 0.4) (layers "F.Cu" "B.Cu") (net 24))
 (via (at 52.121469 83.3) (size 0.8) (drill 0.4) (layers "F.Cu" "B.Cu") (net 24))
 (via (at 46.2 83.3) (size 0.8) (drill 0.4) (layers "F.Cu" "B.Cu") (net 24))
 (segment (start 52.121469 83.3) (end 57.421469 83.3) (width 0.5) (layer "B.Cu") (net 24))
 (segment (start 46.2 56) (end 46.2 83.3) (width 1) (layer "B.Cu") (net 24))
 (segment (start 52.121469 80.3) (end 57.421469 80.3) (width 0.5) (layer "F.Cu") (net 17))
 (segment (start 48.6 97) (end 40.05 97) (width 1) (layer "F.Cu") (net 17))
 (segment (start 34.45 98.5) (end 35.95 97) (width 0.5) (layer "F.Cu") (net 17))
 (segment (start 52.121469 80.3) (end 48.6 80.3) (width 1) (layer "F.Cu") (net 17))
 (segment (start 35.95 97) (end 40.05 97) (width 0.5) (layer "F.Cu") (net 17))
 (via (at 52.121469 80.3) (size 0.8) (drill 0.4) (layers "F.Cu" "B.Cu") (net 17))
 (via (at 48.6 80.3) (size 0.8) (drill 0.4) (layers "F.Cu" "B.Cu") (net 17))
 (via (at 48.6 97) (size 0.8) (drill 0.4) (layers "F.Cu" "B.Cu") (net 17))
 (segment (start 48.6 97) (end 48.6 80.3) (width 1) (layer "B.Cu") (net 17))
 (segment (start 38.95 43.9) (end 49.85 43.9) (width 1) (layer "F.Cu") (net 32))
 (segment (start 49.8 74.3) (end 52.221469 74.3) (width 1) (layer "F.Cu") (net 32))
 (via (at 49.85 43.9) (size 0.8) (drill 0.4) (layers "F.Cu" "B.Cu") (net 32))
 (via (at 49.8 74.3) (size 0.8) (drill 0.4) (layers "F.Cu" "B.Cu") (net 32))
 (via (at 52.221469 74.3) (size 0.8) (drill 0.4) (layers "F.Cu" "B.Cu") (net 32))
 (segment (start 49.822438 74.277562) (end 49.8 74.3) (width 1) (layer "B.Cu") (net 32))
 (segment (start 52.221469 74.3) (end 57.421469 74.3) (width 0.5) (layer "B.Cu") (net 32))
 (segment (start 49.822438 43.927562) (end 49.822438 74.277562) (width 1) (layer "B.Cu") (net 32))
 (segment (start 49.85 43.9) (end 49.822438 43.927562) (width 1) (layer "B.Cu") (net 32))
 (segment (start 69.45 86.3) (end 65.421469 86.3) (width 1) (layer "F.Cu") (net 5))
 (segment (start 52.75 118) (end 39.75 118) (width 1) (layer "F.Cu") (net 5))
 (segment (start 35.95 118) (end 39.75 118) (width 0.5) (layer "F.Cu") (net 5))
 (segment (start 69.5 86.25) (end 69.45 86.3) (width 1) (layer "F.Cu") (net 5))
 (segment (start 34.45 116.5) (end 35.95 118) (width 0.5) (layer "F.Cu") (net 5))
 (via (at 69.5 86.25) (size 0.8) (drill 0.4) (layers "F.Cu" "B.Cu") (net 5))
 (via (at 65.421469 86.3) (size 0.8) (drill 0.4) (layers "F.Cu" "B.Cu") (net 5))
 (via (at 52.75 118) (size 0.8) (drill 0.4) (layers "F.Cu" "B.Cu") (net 5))
 (segment (start 69.5 86.25) (end 69.446378 86.25) (width 1) (layer "B.Cu") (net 5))
 (segment (start 55.954103 99.69952) (end 52.75 102.903623) (width 1) (layer "B.Cu") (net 5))
 (segment (start 65.421469 86.3) (end 60.421469 86.3) (width 0.5) (layer "B.Cu") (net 5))
 (segment (start 52.75 102.903623) (end 52.75 118) (width 1) (layer "B.Cu") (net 5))
 (segment (start 69.446378 86.25) (end 55.996858 99.69952) (width 1) (layer "B.Cu") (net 5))
 (segment (start 55.996858 99.69952) (end 55.954103 99.69952) (width 1) (layer "B.Cu") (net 5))
 (segment (start 56.25 28.8) (end 38.95 28.8) (width 1) (layer "F.Cu") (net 42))
 (segment (start 65.421469 80.3) (end 75.75 80.3) (width 1) (layer "F.Cu") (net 42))
 (via (at 65.421469 80.3) (size 0.8) (drill 0.4) (layers "F.Cu" "B.Cu") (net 42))
 (via (at 75.75 80.3) (size 0.8) (drill 0.4) (layers "F.Cu" "B.Cu") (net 42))
 (via (at 56.25 28.8) (size 0.8) (drill 0.4) (layers "F.Cu" "B.Cu") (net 42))
 (segment (start 56.09952 37.403143) (end 75.75 57.053623) (width 1) (layer "B.Cu") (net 42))
 (segment (start 56.09952 28.95048) (end 56.09952 37.403143) (width 1) (layer "B.Cu") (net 42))
 (segment (start 56.25 28.8) (end 56.09952 28.95048) (width 1) (layer "B.Cu") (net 42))
 (segment (start 75.75 57.053623) (end 75.75 80.3) (width 1) (layer "B.Cu") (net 42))
 (segment (start 65.421469 80.3) (end 60.421469 80.3) (width 0.5) (layer "B.Cu") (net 42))
 (segment (start 73.4005 77.25) (end 73.3505 77.3) (width 1) (layer "F.Cu") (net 71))
 (segment (start 65.421469 77.3) (end 60.421469 77.3) (width 0.5) (layer "F.Cu") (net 71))
 (segment (start 73.3505 77.3) (end 65.421469 77.3) (width 1) (layer "F.Cu") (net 71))
 (via (at 73.4005 77.25) (size 0.8) (drill 0.4) (layers "F.Cu" "B.Cu") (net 71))
 (via (at 65.421469 77.3) (size 0.8) (drill 0.4) (layers "F.Cu" "B.Cu") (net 71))
 (segment (start 72 74.25) (end 71.95 74.3) (width 1) (layer "F.Cu") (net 72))
 (segment (start 71.95 74.3) (end 65.421469 74.3) (width 1) (layer "F.Cu") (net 72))
 (via (at 72 74.25) (size 0.8) (drill 0.4) (layers "F.Cu" "B.Cu") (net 72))
 (via (at 65.421469 74.3) (size 0.8) (drill 0.4) (layers "F.Cu" "B.Cu") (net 72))
 (segment (start 65.421469 74.3) (end 60.421469 74.3) (width 0.5) (layer "B.Cu") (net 72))
 (segment (start 70.75 71.3) (end 65.421469 71.3) (width 1) (layer "F.Cu") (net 43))
 (segment (start 52.200489 23.700489) (end 36.049511 23.700489) (width 1) (layer "F.Cu") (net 43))
 (segment (start 36.049511 23.700489) (end 34.45 25.3) (width 1) (layer "F.Cu") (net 43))
 (segment (start 52.25 23.75) (end 52.200489 23.700489) (width 1) (layer "F.Cu") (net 43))
 (segment (start 65.421469 71.3) (end 60.421469 71.3) (width 0.5) (layer "F.Cu") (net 43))
 (via (at 52.25 23.75) (size 0.8) (drill 0.4) (layers "F.Cu" "B.Cu") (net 43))
 (via (at 65.421469 71.3) (size 0.8) (drill 0.4) (layers "F.Cu" "B.Cu") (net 43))
 (via (at 70.75 71.3) (size 0.8) (drill 0.4) (layers "F.Cu" "B.Cu") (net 43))
 (segment (start 52.24904 23.75096) (end 52.24904 46.702664) (width 1) (layer "B.Cu") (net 43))
 (segment (start 52.24904 46.702664) (end 70.75 65.203623) (width 1) (layer "B.Cu") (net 43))
 (segment (start 52.25 23.75) (end 52.24904 23.75096) (width 1) (layer "B.Cu") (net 43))
 (segment (start 70.75 65.203623) (end 70.75 71.3) (width 1) (layer "B.Cu") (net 43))
 (segment (start 35.95 39.4) (end 34.45 37.9) (width 0.5) (layer "F.Cu") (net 35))
 (segment (start 50.9 39.4) (end 40 39.4) (width 1) (layer "F.Cu") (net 35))
 (segment (start 39.85 39.4) (end 35.95 39.4) (width 0.5) (layer "F.Cu") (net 35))
 (segment (start 51 39.5) (end 50.9 39.4) (width 1) (layer "F.Cu") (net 35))
 (segment (start 68.25 68.3) (end 65.421469 68.3) (width 1) (layer "F.Cu") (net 35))
 (segment (start 40 39.25) (end 39.85 39.4) (width 0.5) (layer "F.Cu") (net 35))
 (via (at 65.421469 68.3) (size 0.8) (drill 0.4) (layers "F.Cu" "B.Cu") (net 35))
 (via (at 51 39.5) (size 0.8) (drill 0.4) (layers "F.Cu" "B.Cu") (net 35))
 (via (at 68.25 68.3) (size 0.8) (drill 0.4) (layers "F.Cu" "B.Cu") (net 35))
 (segment (start 65.421469 68.3) (end 60.421469 68.3) (width 0.5) (layer "B.Cu") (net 35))
 (segment (start 51 39.5) (end 51.04952 39.54952) (width 1) (layer "B.Cu") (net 35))
 (segment (start 51.04952 39.54952) (end 51.04952 49.231673) (width 1) (layer "B.Cu") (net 35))
 (segment (start 51.04952 49.231673) (end 68.25 66.432153) (width 1) (layer "B.Cu") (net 35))
 (segment (start 68.25 66.432153) (end 68.25 68.3) (width 1) (layer "B.Cu") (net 35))
 (segment (start 69.7 87.8) (end 62.921469 87.8) (width 1) (layer "F.Cu") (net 2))
 (segment (start 69.75 87.75) (end 69.7 87.8) (width 1) (layer "F.Cu") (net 2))
 (segment (start 53.65 123.1) (end 38.95 123.1) (width 1) (layer "F.Cu") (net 2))
 (segment (start 53.75 123) (end 53.65 123.1) (width 1) (layer "F.Cu") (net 2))
 (via (at 69.75 87.75) (size 0.8) (drill 0.4) (layers "F.Cu" "B.Cu") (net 2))
 (via (at 53.75 123) (size 0.8) (drill 0.4) (layers "F.Cu" "B.Cu") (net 2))
 (segment (start 69.75 87.75) (end 69.642756 87.75) (width 1) (layer "B.Cu") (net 2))
 (segment (start 56.450961 100.89904) (end 53.94952 103.400481) (width 1) (layer "B.Cu") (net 2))
 (segment (start 69.642756 87.75) (end 56.493716 100.89904) (width 1) (layer "B.Cu") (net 2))
 (segment (start 53.94952 118.496857) (end 53.75 118.696377) (width 1) (layer "B.Cu") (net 2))
 (segment (start 53.75 118.696377) (end 53.75 123) (width 1) (layer "B.Cu") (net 2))
 (segment (start 56.493716 100.89904) (end 56.450961 100.89904) (width 1) (layer "B.Cu") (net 2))
 (segment (start 53.94952 103.400481) (end 53.94952 118.496857) (width 1) (layer "B.Cu") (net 2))
 (segment (start 62.921469 78.8) (end 74.5 78.8) (width 1) (layer "F.Cu") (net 36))
 (segment (start 54.75 37.9) (end 38.95 37.9) (width 1) (layer "F.Cu") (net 36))
 (via (at 54.75 37.9) (size 0.8) (drill 0.4) (layers "F.Cu" "B.Cu") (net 36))
 (via (at 74.5 78.8) (size 0.8) (drill 0.4) (layers "F.Cu" "B.Cu") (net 36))
 (segment (start 54.9 37.9) (end 74.5 57.5) (width 1) (layer "B.Cu") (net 36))
 (segment (start 74.5 57.5) (end 74.5 78.8) (width 1) (layer "B.Cu") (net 36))
 (segment (start 54.75 37.9) (end 54.9 37.9) (width 1) (layer "B.Cu") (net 36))
 (segment (start 73.25 75.75) (end 73.2 75.8) (width 1) (layer "F.Cu") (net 37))
 (segment (start 53.5 36.3) (end 40.1 36.3) (width 1) (layer "F.Cu") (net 37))
 (segment (start 73.2 75.8) (end 62.921469 75.8) (width 1) (layer "F.Cu") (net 37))
 (segment (start 35.9 36.35) (end 34.45 34.9) (width 0.5) (layer "F.Cu") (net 37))
 (segment (start 40.1 36.3) (end 40.05 36.35) (width 0.5) (layer "F.Cu") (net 37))
 (segment (start 40.05 36.35) (end 35.9 36.35) (width 0.5) (layer "F.Cu") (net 37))
 (via (at 53.5 36.3) (size 0.8) (drill 0.4) (layers "F.Cu" "B.Cu") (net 37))
 (via (at 73.25 75.75) (size 0.8) (drill 0.4) (layers "F.Cu" "B.Cu") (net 37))
 (segment (start 53.5 44.25) (end 53.5 36.3) (width 1) (layer "B.Cu") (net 37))
 (segment (start 73.25 75.75) (end 73.25 64) (width 1) (layer "B.Cu") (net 37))
 (segment (start 73.25 64) (end 53.5 44.25) (width 1) (layer "B.Cu") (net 37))
 (segment (start 71.95 72.8) (end 62.921469 72.8) (width 1) (layer "F.Cu") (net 25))
 (segment (start 34.45 52.9) (end 35.95 51.4) (width 0.5) (layer "F.Cu") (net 25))
 (segment (start 58.6 51.4) (end 39.8 51.4) (width 1) (layer "F.Cu") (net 25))
 (segment (start 72 72.75) (end 71.95 72.8) (width 1) (layer "F.Cu") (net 25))
 (segment (start 35.95 51.4) (end 39.8 51.4) (width 0.5) (layer "F.Cu") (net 25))
 (segment (start 58.75 51.25) (end 58.6 51.4) (width 1) (layer "F.Cu") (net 25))
 (via (at 72 72.75) (size 0.8) (drill 0.4) (layers "F.Cu" "B.Cu") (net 25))
 (via (at 58.75 51.25) (size 0.8) (drill 0.4) (layers "F.Cu" "B.Cu") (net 25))
 (segment (start 58.75 51.25) (end 71.94952 64.44952) (width 1) (layer "B.Cu") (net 25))
 (segment (start 71.94952 72.69952) (end 72 72.75) (width 1) (layer "B.Cu") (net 25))
 (segment (start 71.94952 64.44952) (end 71.94952 72.69952) (width 1) (layer "B.Cu") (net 25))
 (segment (start 52.25 48.4) (end 39.6 48.4) (width 1) (layer "F.Cu") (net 27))
 (segment (start 69.45 69.8) (end 62.921469 69.8) (width 1) (layer "F.Cu") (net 27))
 (segment (start 35.95 48.4) (end 34.45 49.9) (width 0.5) (layer "F.Cu") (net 27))
 (segment (start 39.6 48.4) (end 35.95 48.4) (width 0.5) (layer "F.Cu") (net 27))
 (segment (start 69.5 69.75) (end 69.45 69.8) (width 1) (layer "F.Cu") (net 27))
 (via (at 69.5 69.75) (size 0.8) (drill 0.4) (layers "F.Cu" "B.Cu") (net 27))
 (via (at 52.25 48.4) (size 0.8) (drill 0.4) (layers "F.Cu" "B.Cu") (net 27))
 (segment (start 69.44952 65.935295) (end 52.25 48.735775) (width 1) (layer "B.Cu") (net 27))
 (segment (start 52.25 48.735775) (end 52.25 48.4) (width 1) (layer "B.Cu") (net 27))
 (segment (start 69.44952 69.69952) (end 69.44952 65.935295) (width 1) (layer "B.Cu") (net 27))
 (segment (start 69.5 69.75) (end 69.44952 69.69952) (width 1) (layer "B.Cu") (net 27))
 (segment (start 57 27.25) (end 56.950489 27.200489) (width 1) (layer "F.Cu") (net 41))
 (segment (start 76.75 83.25) (end 76.7 83.3) (width 1) (layer "F.Cu") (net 41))
 (segment (start 65.421469 83.3) (end 60.421469 83.3) (width 0.5) (layer "F.Cu") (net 41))
 (segment (start 76.7 83.3) (end 65.421469 83.3) (width 1) (layer "F.Cu") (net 41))
 (segment (start 56.950489 27.200489) (end 36.049511 27.200489) (width 1) (layer "F.Cu") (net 41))
 (segment (start 36.049511 27.200489) (end 34.45 28.8) (width 1) (layer "F.Cu") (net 41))
 (via (at 76.75 83.25) (size 0.8) (drill 0.4) (layers "F.Cu" "B.Cu") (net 41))
 (via (at 57 27.25) (size 0.8) (drill 0.4) (layers "F.Cu" "B.Cu") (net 41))
 (via (at 65.421469 83.3) (size 0.8) (drill 0.4) (layers "F.Cu" "B.Cu") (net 41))
 (segment (start 76.94952 56.556766) (end 57.44952 37.056765) (width 1) (layer "B.Cu") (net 41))
 (segment (start 57.44952 27.69952) (end 57 27.25) (width 1) (layer "B.Cu") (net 41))
 (segment (start 57.44952 37.056765) (end 57.44952 27.69952) (width 1) (layer "B.Cu") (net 41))
 (segment (start 76.75 83.25) (end 76.94952 83.05048) (width 1) (layer "B.Cu") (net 41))
 (segment (start 76.94952 83.05048) (end 76.94952 56.556766) (width 1) (layer "B.Cu") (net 41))
 (segment (start 55.5 98.5) (end 38.95 98.5) (width 1) (layer "F.Cu") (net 18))
 (via (at 55.5 98.5) (size 0.8) (drill 0.4) (layers "F.Cu" "B.Cu") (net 18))
 (via (at 65.421469 65.3) (size 0.8) (drill 0.4) (layers "F.Cu" "B.Cu") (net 18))
 (segment (start 55.5 98.5) (end 66.9 87.1) (width 1) (layer "B.Cu") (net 18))
 (segment (start 65.421469 65.3) (end 60.421469 65.3) (width 0.5) (layer "B.Cu") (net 18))
 (segment (start 66.9 66.778531) (end 65.421469 65.3) (width 1) (layer "B.Cu") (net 18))
 (segment (start 66.9 87.1) (end 66.9 66.778531) (width 1) (layer "B.Cu") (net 18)))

